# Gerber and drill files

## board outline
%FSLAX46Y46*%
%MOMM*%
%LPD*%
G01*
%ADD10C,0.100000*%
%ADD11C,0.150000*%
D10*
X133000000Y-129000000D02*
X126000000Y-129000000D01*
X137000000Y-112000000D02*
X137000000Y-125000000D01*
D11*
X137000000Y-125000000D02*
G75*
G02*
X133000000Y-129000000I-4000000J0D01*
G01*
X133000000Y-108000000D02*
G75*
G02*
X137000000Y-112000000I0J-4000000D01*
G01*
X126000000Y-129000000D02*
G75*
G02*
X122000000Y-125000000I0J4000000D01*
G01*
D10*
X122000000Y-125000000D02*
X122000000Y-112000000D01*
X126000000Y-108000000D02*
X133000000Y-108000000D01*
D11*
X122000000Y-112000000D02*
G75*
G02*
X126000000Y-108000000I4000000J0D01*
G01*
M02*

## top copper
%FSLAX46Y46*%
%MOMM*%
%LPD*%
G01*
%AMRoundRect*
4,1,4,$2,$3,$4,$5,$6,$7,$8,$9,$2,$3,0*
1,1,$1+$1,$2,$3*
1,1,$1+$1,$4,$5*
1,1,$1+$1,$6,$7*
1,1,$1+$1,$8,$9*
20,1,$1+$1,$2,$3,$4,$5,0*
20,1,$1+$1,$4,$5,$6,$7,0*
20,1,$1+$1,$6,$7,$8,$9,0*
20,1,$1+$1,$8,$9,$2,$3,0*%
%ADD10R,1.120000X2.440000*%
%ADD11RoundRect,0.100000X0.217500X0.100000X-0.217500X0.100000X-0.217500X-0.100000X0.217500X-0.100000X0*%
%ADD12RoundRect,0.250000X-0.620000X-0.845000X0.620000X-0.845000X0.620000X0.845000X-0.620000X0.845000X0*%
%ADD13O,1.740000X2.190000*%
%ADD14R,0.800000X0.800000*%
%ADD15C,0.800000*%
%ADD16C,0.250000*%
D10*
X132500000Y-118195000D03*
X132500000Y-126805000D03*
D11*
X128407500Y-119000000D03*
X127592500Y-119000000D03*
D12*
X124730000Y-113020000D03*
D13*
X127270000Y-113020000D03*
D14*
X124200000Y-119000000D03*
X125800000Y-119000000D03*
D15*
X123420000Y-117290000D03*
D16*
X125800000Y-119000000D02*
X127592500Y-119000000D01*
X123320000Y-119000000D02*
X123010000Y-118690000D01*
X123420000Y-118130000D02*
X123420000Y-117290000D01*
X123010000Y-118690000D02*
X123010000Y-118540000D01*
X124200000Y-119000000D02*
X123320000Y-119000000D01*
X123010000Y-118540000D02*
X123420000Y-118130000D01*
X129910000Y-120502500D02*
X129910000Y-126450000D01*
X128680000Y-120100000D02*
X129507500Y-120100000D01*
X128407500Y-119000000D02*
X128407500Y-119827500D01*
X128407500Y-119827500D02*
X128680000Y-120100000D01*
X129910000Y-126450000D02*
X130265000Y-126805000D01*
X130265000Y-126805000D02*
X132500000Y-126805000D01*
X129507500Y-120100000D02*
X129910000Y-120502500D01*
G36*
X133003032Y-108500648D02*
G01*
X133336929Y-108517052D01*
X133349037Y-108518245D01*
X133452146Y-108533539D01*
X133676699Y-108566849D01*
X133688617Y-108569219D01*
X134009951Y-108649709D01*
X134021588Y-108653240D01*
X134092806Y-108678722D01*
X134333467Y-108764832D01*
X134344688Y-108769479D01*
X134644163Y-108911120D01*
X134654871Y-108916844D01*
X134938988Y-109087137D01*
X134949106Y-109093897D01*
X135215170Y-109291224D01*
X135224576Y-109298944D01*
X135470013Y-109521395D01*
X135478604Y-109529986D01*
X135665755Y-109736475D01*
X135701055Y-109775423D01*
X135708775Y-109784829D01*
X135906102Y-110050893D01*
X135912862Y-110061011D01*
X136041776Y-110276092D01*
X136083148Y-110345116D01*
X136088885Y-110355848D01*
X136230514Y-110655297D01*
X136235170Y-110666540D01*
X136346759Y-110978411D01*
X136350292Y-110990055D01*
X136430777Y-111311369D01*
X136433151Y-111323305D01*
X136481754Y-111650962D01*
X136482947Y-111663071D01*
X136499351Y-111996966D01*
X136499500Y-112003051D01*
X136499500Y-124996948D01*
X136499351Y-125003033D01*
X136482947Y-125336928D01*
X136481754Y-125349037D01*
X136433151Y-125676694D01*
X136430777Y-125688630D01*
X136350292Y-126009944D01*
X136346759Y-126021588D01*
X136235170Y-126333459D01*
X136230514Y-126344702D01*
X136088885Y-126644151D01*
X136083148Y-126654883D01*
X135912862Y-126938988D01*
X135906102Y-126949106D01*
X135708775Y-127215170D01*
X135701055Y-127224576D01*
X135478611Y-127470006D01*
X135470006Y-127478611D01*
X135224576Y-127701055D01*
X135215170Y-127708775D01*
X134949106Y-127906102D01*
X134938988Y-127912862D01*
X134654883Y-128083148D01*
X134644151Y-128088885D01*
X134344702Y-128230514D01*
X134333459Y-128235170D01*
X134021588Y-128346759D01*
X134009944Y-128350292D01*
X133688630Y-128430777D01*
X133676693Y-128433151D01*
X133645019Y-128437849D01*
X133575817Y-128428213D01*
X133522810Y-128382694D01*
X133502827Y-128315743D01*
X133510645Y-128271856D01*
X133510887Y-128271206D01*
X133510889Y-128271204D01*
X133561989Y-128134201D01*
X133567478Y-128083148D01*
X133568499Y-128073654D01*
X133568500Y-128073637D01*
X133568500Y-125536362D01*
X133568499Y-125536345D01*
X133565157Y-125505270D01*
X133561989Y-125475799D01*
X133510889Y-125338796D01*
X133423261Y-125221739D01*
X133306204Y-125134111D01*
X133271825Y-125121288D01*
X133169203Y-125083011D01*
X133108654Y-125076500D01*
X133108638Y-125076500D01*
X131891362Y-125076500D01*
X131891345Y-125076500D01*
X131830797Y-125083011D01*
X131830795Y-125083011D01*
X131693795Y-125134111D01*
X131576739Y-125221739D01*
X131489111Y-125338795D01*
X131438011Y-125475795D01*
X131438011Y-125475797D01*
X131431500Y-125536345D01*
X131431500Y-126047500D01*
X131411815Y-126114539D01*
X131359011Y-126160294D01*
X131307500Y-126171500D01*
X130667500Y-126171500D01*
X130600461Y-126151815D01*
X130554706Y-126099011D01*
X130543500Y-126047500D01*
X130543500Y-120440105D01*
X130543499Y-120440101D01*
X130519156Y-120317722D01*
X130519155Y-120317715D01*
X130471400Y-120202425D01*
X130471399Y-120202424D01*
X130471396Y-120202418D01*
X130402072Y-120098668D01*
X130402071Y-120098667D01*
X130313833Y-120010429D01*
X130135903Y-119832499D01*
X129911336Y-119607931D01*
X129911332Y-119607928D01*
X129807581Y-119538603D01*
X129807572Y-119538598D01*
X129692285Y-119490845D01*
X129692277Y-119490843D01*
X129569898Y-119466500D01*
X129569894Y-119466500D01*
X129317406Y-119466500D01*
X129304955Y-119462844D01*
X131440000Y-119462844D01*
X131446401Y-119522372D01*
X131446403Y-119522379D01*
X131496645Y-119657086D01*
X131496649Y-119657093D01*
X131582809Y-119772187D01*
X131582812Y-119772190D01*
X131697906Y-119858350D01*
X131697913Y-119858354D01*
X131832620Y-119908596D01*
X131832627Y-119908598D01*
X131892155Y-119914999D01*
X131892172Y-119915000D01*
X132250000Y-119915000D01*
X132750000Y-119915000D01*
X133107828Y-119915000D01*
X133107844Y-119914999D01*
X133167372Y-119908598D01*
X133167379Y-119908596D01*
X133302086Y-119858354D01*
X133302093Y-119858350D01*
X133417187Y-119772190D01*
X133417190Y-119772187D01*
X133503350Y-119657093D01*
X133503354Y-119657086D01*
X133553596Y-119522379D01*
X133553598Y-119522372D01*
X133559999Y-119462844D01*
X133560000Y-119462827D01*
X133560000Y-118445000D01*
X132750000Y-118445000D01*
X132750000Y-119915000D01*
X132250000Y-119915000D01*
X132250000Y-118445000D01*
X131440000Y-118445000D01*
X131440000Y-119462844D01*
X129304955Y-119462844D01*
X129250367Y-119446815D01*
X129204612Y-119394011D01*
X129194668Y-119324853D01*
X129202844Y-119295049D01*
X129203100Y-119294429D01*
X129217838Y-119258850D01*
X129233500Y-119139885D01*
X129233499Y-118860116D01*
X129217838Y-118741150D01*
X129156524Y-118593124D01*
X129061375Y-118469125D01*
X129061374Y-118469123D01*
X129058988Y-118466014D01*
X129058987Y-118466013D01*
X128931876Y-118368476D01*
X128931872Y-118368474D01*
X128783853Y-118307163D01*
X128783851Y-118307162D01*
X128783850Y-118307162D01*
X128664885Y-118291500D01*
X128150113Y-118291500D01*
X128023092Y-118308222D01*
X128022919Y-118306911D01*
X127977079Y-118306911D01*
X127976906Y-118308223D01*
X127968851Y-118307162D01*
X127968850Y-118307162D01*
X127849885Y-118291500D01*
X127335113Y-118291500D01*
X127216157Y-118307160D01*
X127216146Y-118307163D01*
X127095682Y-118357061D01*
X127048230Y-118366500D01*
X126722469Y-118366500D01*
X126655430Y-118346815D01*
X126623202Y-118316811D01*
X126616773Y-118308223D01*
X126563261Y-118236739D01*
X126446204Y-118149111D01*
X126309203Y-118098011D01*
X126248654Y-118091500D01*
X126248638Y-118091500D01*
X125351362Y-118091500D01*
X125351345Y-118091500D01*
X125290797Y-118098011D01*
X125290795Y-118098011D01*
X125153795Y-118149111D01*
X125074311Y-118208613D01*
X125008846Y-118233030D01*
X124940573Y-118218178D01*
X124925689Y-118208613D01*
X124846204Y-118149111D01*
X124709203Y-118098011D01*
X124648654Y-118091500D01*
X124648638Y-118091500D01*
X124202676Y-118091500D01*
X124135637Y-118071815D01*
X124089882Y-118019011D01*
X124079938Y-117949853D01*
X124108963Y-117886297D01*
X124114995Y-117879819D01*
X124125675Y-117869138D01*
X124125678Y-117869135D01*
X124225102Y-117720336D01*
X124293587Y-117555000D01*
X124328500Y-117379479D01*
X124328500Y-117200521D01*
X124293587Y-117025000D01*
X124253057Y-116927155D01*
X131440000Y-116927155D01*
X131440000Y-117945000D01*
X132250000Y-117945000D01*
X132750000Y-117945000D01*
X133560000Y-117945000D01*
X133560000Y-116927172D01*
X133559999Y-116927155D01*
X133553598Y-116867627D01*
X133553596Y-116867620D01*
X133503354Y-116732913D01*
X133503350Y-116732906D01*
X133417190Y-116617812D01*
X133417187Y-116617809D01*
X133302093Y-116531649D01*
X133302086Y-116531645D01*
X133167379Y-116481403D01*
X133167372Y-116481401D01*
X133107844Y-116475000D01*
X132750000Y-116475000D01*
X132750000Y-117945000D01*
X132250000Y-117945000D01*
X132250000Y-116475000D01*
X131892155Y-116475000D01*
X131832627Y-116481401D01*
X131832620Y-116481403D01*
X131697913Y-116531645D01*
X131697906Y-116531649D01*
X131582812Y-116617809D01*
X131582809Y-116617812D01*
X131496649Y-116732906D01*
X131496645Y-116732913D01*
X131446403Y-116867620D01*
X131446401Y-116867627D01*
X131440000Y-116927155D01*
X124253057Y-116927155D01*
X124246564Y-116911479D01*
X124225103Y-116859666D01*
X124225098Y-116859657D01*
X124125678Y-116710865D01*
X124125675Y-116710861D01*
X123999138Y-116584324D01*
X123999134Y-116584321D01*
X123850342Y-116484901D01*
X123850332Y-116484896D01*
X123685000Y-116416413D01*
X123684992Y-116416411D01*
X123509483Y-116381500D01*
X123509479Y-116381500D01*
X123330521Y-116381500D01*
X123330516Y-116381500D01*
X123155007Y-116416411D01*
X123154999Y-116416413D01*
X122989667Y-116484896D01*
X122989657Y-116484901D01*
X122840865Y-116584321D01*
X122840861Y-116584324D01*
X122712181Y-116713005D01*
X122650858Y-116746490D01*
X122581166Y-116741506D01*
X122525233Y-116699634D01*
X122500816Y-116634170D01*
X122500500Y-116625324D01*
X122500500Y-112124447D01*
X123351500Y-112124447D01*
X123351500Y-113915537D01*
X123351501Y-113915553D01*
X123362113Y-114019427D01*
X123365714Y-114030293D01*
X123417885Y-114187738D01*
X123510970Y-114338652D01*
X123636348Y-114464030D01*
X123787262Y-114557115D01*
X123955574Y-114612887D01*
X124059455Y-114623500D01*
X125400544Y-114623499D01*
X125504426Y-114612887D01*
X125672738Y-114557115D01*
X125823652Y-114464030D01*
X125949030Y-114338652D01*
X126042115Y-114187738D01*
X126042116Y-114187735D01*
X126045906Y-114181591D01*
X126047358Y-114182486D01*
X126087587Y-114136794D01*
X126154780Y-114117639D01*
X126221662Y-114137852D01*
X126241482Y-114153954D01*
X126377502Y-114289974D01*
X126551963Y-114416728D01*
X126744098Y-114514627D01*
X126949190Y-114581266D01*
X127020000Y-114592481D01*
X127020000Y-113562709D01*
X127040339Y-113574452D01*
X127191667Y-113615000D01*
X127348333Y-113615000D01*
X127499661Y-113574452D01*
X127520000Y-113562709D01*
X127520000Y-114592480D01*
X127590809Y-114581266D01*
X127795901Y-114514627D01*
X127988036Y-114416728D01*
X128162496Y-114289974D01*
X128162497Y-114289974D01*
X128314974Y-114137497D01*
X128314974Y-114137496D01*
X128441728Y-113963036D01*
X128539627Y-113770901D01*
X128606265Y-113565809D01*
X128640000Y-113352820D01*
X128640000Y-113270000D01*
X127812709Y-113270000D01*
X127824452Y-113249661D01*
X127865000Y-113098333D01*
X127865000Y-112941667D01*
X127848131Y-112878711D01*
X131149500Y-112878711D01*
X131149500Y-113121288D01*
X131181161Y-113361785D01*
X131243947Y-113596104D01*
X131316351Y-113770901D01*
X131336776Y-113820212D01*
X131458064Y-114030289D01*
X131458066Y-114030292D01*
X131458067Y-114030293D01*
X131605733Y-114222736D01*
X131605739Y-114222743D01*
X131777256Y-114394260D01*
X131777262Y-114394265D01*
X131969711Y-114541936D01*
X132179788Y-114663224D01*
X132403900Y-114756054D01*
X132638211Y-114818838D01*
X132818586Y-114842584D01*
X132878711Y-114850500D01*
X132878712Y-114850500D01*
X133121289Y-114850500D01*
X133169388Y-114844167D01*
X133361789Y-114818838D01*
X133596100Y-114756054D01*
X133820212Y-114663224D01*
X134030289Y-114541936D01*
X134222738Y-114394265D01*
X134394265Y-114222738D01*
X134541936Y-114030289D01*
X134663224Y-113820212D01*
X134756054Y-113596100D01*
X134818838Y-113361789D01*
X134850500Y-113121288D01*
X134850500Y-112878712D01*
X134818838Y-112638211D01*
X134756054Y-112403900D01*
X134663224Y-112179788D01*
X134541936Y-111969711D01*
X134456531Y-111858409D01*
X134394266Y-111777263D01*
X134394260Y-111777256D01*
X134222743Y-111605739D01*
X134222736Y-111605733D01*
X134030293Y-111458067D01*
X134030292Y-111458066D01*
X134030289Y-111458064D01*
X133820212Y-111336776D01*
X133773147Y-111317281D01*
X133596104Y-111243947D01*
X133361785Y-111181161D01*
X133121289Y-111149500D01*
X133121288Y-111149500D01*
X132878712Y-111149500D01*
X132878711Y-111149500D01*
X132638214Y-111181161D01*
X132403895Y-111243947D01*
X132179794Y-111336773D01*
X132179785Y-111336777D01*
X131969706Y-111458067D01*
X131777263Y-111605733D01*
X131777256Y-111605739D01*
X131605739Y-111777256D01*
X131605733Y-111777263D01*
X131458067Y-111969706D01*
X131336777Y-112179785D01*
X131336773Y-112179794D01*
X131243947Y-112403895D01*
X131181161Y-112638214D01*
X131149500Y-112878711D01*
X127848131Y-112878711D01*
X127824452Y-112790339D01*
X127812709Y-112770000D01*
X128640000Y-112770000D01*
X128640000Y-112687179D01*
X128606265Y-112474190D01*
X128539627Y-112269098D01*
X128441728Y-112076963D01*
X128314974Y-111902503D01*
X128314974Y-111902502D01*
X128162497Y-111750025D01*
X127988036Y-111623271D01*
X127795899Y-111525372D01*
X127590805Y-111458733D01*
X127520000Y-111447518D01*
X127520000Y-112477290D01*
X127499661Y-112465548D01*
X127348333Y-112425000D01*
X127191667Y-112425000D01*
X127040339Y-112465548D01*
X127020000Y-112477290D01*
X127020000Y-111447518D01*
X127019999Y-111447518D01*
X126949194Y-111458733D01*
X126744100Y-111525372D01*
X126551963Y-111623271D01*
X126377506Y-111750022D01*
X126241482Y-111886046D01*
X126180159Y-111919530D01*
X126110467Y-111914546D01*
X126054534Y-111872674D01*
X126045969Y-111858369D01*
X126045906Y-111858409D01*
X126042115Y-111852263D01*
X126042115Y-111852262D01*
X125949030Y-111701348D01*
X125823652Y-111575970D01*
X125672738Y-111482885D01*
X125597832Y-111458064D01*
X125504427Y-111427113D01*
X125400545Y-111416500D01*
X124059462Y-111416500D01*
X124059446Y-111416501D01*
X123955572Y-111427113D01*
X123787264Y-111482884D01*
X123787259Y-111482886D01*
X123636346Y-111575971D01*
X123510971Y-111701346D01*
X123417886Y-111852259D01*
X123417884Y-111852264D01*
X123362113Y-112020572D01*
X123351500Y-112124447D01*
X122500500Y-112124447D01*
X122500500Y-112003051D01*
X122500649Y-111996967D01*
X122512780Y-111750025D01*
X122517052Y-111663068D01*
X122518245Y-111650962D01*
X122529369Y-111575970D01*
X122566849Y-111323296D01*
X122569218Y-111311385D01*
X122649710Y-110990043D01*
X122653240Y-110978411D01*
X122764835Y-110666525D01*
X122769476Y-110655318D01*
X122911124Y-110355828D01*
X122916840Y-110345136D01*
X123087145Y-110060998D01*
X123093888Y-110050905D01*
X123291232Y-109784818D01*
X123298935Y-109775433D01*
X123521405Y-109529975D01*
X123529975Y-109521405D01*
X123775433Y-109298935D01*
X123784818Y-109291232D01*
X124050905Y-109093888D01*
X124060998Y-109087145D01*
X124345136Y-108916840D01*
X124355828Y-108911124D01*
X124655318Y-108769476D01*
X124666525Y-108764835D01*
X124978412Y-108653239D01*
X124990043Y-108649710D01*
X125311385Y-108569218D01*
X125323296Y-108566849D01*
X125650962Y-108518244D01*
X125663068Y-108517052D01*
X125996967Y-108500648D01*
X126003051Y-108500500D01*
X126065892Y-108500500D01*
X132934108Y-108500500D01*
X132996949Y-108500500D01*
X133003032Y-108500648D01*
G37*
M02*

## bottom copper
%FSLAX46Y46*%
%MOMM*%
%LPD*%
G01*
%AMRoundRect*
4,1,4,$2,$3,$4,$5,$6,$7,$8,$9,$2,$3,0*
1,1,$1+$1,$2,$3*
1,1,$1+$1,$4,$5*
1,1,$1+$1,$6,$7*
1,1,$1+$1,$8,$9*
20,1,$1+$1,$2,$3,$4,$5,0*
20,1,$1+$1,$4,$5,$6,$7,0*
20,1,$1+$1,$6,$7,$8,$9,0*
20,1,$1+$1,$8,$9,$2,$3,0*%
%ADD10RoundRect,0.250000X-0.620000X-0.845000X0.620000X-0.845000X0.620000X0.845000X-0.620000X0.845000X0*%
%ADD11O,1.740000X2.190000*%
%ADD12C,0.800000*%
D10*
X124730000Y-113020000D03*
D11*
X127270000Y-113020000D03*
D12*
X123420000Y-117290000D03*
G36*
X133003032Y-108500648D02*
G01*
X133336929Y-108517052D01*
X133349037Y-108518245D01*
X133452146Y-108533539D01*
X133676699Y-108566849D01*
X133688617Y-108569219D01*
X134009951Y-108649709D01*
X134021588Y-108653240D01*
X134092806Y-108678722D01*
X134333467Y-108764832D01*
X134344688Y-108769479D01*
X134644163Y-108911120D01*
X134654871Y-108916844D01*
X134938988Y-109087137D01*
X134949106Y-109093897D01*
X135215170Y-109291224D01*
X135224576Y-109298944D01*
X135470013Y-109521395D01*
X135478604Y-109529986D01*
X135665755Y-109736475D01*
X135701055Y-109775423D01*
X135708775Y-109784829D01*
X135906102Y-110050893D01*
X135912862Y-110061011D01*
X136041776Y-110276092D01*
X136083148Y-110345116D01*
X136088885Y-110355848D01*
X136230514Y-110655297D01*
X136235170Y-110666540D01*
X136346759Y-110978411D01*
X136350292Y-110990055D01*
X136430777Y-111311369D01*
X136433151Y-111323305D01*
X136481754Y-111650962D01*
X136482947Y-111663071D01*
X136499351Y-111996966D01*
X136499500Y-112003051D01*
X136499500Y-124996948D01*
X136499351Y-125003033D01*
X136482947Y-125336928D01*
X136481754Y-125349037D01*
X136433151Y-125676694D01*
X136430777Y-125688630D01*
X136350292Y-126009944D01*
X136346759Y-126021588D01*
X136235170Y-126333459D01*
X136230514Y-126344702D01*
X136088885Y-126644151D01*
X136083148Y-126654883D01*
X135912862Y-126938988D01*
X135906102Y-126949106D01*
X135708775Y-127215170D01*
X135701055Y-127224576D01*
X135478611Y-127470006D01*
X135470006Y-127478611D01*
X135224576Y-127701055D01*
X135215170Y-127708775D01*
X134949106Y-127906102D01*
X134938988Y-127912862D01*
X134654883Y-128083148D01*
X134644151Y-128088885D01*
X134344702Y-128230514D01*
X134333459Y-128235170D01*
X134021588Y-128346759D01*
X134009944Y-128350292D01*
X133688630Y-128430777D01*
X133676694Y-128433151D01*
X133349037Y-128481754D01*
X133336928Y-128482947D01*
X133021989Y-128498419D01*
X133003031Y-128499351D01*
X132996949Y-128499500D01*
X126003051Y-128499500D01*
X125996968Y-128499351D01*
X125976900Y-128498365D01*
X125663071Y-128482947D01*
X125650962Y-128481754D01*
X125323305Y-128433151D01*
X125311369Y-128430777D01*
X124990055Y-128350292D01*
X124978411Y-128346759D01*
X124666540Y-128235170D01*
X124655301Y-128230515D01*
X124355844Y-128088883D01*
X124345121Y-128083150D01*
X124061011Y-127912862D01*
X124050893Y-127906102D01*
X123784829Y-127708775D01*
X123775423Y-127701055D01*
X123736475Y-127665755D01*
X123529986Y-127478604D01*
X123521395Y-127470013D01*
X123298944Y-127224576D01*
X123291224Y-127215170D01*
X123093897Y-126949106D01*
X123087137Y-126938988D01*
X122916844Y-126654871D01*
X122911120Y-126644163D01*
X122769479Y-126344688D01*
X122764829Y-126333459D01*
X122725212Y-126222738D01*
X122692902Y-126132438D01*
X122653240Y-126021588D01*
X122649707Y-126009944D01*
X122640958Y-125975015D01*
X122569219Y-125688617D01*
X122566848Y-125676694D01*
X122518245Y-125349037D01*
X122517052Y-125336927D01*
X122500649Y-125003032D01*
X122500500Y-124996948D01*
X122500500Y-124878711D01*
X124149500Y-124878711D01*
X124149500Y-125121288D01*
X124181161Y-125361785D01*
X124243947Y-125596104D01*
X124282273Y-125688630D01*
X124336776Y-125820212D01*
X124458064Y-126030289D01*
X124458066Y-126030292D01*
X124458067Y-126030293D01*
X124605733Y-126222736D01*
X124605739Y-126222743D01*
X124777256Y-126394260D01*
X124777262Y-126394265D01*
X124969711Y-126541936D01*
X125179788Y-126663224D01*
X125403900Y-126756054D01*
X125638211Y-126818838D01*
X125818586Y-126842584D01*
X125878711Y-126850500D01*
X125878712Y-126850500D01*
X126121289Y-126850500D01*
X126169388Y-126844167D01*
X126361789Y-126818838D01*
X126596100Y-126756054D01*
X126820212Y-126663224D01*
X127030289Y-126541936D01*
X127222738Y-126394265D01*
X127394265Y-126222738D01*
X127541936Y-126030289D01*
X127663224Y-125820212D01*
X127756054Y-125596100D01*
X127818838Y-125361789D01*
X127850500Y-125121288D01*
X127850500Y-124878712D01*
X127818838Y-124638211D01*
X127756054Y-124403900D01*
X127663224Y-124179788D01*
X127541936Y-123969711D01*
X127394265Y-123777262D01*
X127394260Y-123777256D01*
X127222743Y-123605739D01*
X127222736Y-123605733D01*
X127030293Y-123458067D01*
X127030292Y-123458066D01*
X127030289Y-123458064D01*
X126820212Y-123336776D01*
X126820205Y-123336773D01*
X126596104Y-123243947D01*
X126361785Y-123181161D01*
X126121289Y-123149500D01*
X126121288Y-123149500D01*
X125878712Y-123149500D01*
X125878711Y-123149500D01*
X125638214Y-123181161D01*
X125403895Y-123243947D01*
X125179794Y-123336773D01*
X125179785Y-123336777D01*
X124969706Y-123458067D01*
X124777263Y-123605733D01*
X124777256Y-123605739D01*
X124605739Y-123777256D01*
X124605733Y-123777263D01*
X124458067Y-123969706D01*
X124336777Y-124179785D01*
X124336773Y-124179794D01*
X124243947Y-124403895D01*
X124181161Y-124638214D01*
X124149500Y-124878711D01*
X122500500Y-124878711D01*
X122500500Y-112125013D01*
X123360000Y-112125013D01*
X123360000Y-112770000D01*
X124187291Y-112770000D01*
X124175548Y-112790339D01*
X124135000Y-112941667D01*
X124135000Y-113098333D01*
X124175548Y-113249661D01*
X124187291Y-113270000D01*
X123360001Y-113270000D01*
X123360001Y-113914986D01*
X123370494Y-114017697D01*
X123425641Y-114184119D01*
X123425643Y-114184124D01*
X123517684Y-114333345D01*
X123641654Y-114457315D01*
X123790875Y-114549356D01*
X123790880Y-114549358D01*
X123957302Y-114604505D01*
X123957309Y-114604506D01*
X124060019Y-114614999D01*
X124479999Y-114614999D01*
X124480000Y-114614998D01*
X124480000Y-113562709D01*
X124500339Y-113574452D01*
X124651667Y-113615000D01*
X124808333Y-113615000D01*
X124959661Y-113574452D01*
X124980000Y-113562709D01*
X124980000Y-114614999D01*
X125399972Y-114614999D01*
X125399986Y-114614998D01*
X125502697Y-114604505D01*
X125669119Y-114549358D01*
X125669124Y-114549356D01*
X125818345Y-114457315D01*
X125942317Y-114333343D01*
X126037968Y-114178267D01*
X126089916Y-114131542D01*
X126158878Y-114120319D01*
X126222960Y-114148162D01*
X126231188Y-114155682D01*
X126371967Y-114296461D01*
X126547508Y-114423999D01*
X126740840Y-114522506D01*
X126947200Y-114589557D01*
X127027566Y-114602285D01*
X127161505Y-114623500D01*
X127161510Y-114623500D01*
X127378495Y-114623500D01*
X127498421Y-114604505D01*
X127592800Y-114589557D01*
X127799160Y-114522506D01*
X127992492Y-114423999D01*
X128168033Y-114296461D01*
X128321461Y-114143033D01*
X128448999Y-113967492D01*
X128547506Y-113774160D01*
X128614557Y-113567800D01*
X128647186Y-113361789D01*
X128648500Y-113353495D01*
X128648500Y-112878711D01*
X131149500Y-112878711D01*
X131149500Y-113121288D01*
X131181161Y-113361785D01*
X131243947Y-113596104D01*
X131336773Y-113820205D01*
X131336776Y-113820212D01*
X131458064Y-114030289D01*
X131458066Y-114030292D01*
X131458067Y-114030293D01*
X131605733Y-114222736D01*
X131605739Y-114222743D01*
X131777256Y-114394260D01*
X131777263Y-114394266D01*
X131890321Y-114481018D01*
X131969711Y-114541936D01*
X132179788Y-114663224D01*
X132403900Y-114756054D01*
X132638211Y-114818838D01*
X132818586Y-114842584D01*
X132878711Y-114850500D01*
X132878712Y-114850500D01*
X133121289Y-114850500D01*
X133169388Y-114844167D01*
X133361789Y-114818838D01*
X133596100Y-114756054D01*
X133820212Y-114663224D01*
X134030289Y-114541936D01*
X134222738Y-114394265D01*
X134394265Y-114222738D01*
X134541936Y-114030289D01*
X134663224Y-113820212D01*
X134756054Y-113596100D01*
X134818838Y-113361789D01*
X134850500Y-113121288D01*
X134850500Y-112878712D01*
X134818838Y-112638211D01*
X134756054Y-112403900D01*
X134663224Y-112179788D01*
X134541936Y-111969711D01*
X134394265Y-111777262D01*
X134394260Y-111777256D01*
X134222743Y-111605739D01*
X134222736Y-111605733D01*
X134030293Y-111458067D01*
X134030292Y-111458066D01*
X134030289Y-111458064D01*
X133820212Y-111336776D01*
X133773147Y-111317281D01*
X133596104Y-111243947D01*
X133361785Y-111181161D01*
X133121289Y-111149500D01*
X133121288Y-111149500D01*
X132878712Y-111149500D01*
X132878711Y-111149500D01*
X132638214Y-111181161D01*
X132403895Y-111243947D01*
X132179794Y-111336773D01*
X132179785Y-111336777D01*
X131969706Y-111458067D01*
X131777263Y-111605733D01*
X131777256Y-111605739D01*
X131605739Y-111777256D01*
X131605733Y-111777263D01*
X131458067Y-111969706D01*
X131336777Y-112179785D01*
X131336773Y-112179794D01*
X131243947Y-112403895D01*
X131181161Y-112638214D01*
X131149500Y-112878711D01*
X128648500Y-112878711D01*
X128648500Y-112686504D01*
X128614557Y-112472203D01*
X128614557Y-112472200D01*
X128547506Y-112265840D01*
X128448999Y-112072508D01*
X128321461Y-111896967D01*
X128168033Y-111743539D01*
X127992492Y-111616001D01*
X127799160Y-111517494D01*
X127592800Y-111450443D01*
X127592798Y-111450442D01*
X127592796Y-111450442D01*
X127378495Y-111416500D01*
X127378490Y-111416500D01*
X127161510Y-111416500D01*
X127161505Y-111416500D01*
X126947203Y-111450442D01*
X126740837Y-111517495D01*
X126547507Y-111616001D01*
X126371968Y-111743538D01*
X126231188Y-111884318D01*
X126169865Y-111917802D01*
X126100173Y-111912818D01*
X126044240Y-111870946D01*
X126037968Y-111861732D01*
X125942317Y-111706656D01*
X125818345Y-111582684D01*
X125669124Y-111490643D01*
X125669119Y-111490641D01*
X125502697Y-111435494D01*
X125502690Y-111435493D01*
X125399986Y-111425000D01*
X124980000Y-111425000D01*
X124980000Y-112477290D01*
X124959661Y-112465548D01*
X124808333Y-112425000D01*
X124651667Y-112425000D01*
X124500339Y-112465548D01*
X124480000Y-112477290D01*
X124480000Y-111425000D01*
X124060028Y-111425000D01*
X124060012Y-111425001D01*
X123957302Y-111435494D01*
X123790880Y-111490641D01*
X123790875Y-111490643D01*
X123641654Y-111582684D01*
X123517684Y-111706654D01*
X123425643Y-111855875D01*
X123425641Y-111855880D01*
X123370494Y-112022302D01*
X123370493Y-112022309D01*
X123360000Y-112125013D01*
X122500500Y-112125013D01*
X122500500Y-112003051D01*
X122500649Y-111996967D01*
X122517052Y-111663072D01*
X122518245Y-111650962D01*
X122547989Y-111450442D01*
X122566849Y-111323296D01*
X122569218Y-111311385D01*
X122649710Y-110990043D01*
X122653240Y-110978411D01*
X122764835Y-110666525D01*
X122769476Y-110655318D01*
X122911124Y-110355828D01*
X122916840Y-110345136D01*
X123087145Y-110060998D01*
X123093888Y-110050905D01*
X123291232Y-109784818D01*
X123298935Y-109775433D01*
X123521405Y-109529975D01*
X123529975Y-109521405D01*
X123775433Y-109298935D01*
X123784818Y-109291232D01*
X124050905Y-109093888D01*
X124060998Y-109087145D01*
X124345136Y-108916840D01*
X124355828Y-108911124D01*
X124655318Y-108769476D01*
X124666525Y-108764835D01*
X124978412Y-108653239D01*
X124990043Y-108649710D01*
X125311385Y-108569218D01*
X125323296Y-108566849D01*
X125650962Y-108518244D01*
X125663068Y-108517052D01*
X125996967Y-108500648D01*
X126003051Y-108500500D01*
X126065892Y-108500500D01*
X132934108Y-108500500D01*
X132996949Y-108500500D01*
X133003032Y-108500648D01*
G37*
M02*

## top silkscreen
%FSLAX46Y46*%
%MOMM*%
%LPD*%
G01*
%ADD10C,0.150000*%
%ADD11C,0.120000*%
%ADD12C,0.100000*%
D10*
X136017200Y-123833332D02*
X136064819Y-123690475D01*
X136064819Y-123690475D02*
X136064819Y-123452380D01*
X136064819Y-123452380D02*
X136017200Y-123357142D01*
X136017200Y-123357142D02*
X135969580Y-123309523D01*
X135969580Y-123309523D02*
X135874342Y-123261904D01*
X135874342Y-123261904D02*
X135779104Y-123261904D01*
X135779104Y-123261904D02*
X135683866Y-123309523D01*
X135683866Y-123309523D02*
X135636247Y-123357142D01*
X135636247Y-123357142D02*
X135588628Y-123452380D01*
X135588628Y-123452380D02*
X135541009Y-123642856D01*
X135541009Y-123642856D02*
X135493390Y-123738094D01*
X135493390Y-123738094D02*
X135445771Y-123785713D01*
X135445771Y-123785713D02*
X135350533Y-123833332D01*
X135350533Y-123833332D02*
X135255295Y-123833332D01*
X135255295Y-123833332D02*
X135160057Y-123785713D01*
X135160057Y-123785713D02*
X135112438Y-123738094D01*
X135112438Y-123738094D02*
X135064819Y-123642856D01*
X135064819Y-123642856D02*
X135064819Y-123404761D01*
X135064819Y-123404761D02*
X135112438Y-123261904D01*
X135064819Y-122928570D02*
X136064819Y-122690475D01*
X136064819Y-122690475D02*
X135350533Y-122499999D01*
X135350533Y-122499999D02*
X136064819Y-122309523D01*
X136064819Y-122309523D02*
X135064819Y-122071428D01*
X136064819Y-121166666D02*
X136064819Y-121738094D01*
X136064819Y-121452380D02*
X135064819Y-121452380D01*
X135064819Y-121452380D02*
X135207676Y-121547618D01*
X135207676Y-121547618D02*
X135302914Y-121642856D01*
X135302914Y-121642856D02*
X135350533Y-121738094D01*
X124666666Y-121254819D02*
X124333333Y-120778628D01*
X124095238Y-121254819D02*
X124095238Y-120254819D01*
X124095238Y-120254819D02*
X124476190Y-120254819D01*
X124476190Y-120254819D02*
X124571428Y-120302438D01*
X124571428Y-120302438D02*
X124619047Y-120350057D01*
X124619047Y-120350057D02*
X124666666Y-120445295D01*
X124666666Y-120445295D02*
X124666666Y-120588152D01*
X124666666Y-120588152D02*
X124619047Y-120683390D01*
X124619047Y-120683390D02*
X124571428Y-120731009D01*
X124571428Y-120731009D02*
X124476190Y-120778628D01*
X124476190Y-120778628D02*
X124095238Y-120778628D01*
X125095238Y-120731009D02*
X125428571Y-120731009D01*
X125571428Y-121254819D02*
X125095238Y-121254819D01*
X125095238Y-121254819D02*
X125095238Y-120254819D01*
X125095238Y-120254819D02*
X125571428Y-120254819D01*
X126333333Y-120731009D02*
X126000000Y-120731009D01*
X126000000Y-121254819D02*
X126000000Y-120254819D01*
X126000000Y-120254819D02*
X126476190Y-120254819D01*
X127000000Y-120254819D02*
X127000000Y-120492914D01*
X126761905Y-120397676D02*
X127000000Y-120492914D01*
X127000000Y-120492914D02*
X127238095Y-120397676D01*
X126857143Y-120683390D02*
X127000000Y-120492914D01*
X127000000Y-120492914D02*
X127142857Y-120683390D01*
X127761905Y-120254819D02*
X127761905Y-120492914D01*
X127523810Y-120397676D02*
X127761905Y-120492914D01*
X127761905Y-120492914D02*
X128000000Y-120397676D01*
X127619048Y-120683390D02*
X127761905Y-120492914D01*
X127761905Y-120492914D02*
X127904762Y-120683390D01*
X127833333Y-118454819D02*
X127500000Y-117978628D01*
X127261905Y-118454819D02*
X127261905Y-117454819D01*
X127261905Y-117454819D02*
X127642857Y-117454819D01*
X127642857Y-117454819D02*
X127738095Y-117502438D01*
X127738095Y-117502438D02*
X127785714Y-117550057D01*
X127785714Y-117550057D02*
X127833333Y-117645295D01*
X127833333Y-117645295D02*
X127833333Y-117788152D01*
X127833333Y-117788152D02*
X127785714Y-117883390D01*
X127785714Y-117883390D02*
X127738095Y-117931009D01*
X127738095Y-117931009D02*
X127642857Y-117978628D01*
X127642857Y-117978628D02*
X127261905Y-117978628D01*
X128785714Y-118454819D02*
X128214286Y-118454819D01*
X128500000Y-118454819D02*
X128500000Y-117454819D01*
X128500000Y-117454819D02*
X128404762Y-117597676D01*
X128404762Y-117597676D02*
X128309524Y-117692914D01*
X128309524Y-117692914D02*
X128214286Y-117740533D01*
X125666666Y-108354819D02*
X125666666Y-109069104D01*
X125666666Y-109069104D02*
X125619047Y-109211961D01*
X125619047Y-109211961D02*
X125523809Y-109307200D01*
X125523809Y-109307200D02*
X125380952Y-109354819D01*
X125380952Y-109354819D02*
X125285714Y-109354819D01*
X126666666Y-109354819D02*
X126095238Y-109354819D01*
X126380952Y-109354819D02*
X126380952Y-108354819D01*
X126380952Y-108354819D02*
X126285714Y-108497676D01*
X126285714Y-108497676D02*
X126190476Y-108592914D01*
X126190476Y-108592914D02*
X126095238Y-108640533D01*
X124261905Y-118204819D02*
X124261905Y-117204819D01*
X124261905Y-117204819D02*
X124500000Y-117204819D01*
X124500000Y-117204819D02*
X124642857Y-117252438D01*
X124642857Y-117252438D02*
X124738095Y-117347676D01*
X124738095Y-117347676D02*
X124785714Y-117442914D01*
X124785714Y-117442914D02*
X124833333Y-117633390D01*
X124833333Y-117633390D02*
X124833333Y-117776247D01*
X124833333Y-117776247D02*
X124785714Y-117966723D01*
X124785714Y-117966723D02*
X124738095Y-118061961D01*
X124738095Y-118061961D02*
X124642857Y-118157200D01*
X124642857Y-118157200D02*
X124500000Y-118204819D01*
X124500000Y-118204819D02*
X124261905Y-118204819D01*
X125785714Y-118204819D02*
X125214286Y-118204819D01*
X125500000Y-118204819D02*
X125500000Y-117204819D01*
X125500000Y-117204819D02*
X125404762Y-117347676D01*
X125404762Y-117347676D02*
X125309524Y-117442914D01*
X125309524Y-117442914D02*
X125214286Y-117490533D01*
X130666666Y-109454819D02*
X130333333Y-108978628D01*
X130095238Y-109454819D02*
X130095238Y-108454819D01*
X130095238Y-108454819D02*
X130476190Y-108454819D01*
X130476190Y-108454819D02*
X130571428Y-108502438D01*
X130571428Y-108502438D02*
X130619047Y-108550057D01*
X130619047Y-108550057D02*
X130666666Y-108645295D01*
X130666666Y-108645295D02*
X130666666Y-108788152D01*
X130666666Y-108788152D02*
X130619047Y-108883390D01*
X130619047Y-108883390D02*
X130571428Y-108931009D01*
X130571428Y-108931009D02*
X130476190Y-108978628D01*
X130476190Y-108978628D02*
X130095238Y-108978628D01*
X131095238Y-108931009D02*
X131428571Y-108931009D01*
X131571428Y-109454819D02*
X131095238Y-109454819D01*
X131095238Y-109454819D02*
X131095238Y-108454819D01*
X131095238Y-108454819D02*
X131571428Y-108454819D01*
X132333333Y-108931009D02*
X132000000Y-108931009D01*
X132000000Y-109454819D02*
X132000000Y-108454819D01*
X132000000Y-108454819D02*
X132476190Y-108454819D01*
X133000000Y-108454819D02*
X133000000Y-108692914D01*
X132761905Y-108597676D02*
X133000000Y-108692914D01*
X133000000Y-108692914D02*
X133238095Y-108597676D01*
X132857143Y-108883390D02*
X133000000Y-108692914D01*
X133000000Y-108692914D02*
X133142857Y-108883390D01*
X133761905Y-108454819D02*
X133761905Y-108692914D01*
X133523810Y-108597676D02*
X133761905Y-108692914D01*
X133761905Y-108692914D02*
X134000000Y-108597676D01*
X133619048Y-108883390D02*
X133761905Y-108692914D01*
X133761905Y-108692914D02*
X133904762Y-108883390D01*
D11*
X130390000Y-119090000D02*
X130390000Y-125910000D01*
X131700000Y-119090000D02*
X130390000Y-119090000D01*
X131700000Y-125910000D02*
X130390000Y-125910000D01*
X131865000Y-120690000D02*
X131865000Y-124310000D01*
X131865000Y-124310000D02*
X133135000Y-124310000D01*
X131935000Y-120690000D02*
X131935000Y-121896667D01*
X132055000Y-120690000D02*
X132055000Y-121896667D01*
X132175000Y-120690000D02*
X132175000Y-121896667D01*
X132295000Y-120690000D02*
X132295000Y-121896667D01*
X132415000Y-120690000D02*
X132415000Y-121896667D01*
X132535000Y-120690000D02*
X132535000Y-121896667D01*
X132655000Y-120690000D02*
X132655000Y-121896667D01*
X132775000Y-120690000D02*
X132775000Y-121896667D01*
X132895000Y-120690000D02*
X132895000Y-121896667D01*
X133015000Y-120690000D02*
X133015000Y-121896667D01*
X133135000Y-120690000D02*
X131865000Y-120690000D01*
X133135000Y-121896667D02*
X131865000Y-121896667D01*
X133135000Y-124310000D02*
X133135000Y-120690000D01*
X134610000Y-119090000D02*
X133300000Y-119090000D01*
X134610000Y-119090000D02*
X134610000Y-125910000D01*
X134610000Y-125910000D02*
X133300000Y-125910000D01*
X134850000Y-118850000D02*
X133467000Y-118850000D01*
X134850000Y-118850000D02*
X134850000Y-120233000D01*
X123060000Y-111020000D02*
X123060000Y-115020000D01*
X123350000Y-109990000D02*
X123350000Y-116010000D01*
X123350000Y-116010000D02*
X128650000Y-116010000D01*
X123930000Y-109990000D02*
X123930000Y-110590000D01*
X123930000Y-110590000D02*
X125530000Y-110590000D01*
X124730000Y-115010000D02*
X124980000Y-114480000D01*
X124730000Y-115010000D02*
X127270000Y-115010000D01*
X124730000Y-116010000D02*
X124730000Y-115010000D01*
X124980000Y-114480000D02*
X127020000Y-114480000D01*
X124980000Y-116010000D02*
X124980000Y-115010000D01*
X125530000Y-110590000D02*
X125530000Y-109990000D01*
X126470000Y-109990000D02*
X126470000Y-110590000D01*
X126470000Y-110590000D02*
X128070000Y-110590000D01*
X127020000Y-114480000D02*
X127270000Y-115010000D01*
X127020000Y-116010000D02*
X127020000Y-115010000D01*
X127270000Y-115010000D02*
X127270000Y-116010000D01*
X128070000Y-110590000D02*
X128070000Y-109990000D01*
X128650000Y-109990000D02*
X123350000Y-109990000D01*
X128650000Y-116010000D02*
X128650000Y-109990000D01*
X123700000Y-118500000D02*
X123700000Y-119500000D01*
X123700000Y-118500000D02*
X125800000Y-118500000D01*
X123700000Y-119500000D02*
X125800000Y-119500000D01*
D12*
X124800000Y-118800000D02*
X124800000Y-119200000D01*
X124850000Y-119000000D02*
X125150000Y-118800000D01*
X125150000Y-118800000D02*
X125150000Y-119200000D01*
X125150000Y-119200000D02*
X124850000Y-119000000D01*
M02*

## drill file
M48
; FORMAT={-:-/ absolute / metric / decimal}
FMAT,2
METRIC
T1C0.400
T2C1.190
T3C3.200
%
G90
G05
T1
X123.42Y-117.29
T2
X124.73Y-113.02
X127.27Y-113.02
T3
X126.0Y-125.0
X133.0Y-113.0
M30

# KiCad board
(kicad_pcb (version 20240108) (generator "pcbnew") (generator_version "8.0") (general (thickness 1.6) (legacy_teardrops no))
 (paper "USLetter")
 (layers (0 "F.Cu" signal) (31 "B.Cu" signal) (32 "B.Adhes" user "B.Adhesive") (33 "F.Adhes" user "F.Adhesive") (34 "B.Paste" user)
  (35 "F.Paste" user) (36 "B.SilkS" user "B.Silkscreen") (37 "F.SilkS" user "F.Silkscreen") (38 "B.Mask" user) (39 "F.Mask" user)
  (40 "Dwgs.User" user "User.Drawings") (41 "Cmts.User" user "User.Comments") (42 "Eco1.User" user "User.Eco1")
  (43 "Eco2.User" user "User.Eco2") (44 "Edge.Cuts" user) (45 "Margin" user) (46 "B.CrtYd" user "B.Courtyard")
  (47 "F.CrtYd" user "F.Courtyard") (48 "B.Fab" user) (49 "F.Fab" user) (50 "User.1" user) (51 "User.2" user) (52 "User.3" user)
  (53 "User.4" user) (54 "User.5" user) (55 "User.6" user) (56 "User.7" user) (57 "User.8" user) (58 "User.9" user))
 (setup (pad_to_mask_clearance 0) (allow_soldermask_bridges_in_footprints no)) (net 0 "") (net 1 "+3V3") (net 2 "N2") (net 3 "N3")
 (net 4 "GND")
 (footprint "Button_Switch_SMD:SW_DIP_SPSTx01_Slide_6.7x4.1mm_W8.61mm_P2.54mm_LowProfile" (layer "F.Cu") (at 132.5 122.5 -90)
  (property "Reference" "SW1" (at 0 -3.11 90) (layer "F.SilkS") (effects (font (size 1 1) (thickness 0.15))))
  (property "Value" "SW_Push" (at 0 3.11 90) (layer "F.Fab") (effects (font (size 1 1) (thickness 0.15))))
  (fp_line (start -3.41 2.11) (end 3.41 2.11) (stroke (width 0.12) (type solid)) (layer "F.SilkS"))
  (fp_line (start -3.41 0.8) (end -3.41 2.11) (stroke (width 0.12) (type solid)) (layer "F.SilkS"))
  (fp_line (start 3.41 0.8) (end 3.41 2.11) (stroke (width 0.12) (type solid)) (layer "F.SilkS"))
  (fp_line (start -1.81 0.635) (end 1.81 0.635) (stroke (width 0.12) (type solid)) (layer "F.SilkS"))
  (fp_line (start 1.81 0.635) (end 1.81 -0.635) (stroke (width 0.12) (type solid)) (layer "F.SilkS"))
  (fp_line (start -1.81 0.565) (end -0.603333 0.565) (stroke (width 0.12) (type solid)) (layer "F.SilkS"))
  (fp_line (start -1.81 0.445) (end -0.603333 0.445) (stroke (width 0.12) (type solid)) (layer "F.SilkS"))
  (fp_line (start -1.81 0.325) (end -0.603333 0.325) (stroke (width 0.12) (type solid)) (layer "F.SilkS"))
  (fp_line (start -1.81 0.205) (end -0.603333 0.205) (stroke (width 0.12) (type solid)) (layer "F.SilkS"))
  (fp_line (start -1.81 0.085) (end -0.603333 0.085) (stroke (width 0.12) (type solid)) (layer "F.SilkS"))
  (fp_line (start -1.81 -0.035) (end -0.603333 -0.035) (stroke (width 0.12) (type solid)) (layer "F.SilkS"))
  (fp_line (start -1.81 -0.155) (end -0.603333 -0.155) (stroke (width 0.12) (type solid)) (layer "F.SilkS"))
  (fp_line (start -1.81 -0.275) (end -0.603333 -0.275) (stroke (width 0.12) (type solid)) (layer "F.SilkS"))
  (fp_line (start -1.81 -0.395) (end -0.603333 -0.395) (stroke (width 0.12) (type solid)) (layer "F.SilkS"))
  (fp_line (start -1.81 -0.515) (end -0.603333 -0.515) (stroke (width 0.12) (type solid)) (layer "F.SilkS"))
  (fp_line (start -1.81 -0.635) (end -1.81 0.635) (stroke (width 0.12) (type solid)) (layer "F.SilkS"))
  (fp_line (start -0.603333 -0.635) (end -0.603333 0.635) (stroke (width 0.12) (type solid)) (layer "F.SilkS"))
  (fp_line (start 1.81 -0.635) (end -1.81 -0.635) (stroke (width 0.12) (type solid)) (layer "F.SilkS"))
  (fp_line (start -3.41 -2.11) (end -3.41 -0.8) (stroke (width 0.12) (type solid)) (layer "F.SilkS"))
  (fp_line (start -3.41 -2.11) (end 3.41 -2.11) (stroke (width 0.12) (type solid)) (layer "F.SilkS"))
  (fp_line (start 3.41 -2.11) (end 3.41 -0.8) (stroke (width 0.12) (type solid)) (layer "F.SilkS"))
  (fp_line (start -3.65 -2.35) (end -3.65 -0.967) (stroke (width 0.12) (type solid)) (layer "F.SilkS"))
  (fp_line (start -3.65 -2.35) (end -2.267 -2.35) (stroke (width 0.12) (type solid)) (layer "F.SilkS"))
  (pad "1" smd rect (at -4.305 0 270) (size 2.44 1.12) (layers "F.Cu" "F.Paste" "F.Mask") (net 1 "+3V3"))
  (pad "2" smd rect (at 4.305 0 270) (size 2.44 1.12) (layers "F.Cu" "F.Paste" "F.Mask") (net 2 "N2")))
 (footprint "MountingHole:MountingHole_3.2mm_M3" (layer "F.Cu") (at 126 125)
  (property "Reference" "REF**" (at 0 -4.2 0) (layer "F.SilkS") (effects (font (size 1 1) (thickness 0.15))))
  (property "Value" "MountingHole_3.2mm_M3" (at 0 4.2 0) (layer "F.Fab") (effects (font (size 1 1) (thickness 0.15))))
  (pad "" np_thru_hole circle (at 0 0) (size 3.2 3.2) (drill 3.2) (layers "*.Cu" "*.Mask")))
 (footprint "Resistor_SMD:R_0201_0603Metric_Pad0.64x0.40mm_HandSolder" (layer "F.Cu") (at 128 119 180)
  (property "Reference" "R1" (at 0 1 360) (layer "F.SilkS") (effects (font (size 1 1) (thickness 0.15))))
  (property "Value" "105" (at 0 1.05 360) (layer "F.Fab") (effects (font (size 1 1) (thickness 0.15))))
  (pad "" smd roundrect (at -0.4325 0 180) (size 0.458 0.36) (layers "F.Paste") (roundrect_rratio 0.25))
  (pad "" smd roundrect (at 0.4325 0 180) (size 0.458 0.36) (layers "F.Paste") (roundrect_rratio 0.25))
  (pad "1" smd roundrect (at -0.4075 0 180) (size 0.635 0.4) (layers "F.Cu" "F.Mask") (roundrect_rratio 0.25) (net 2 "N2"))
  (pad "2" smd roundrect (at 0.4075 0 180) (size 0.635 0.4) (layers "F.Cu" "F.Mask") (roundrect_rratio 0.25) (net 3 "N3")))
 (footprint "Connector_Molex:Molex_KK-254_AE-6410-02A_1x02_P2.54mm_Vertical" (layer "F.Cu") (at 124.73 113.02)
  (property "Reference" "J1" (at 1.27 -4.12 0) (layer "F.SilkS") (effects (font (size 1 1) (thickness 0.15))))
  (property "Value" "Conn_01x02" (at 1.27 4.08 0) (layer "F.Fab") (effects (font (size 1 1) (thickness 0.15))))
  (fp_line (start -1.67 -2) (end -1.67 2) (stroke (width 0.12) (type solid)) (layer "F.SilkS"))
  (fp_line (start -1.38 -3.03) (end -1.38 2.99) (stroke (width 0.12) (type solid)) (layer "F.SilkS"))
  (fp_line (start -1.38 2.99) (end 3.92 2.99) (stroke (width 0.12) (type solid)) (layer "F.SilkS"))
  (fp_line (start -0.8 -3.03) (end -0.8 -2.43) (stroke (width 0.12) (type solid)) (layer "F.SilkS"))
  (fp_line (start -0.8 -2.43) (end 0.8 -2.43) (stroke (width 0.12) (type solid)) (layer "F.SilkS"))
  (fp_line (start 0 1.99) (end 0.25 1.46) (stroke (width 0.12) (type solid)) (layer "F.SilkS"))
  (fp_line (start 0 1.99) (end 2.54 1.99) (stroke (width 0.12) (type solid)) (layer "F.SilkS"))
  (fp_line (start 0 2.99) (end 0 1.99) (stroke (width 0.12) (type solid)) (layer "F.SilkS"))
  (fp_line (start 0.25 1.46) (end 2.29 1.46) (stroke (width 0.12) (type solid)) (layer "F.SilkS"))
  (fp_line (start 0.25 2.99) (end 0.25 1.99) (stroke (width 0.12) (type solid)) (layer "F.SilkS"))
  (fp_line (start 0.8 -2.43) (end 0.8 -3.03) (stroke (width 0.12) (type solid)) (layer "F.SilkS"))
  (fp_line (start 1.74 -3.03) (end 1.74 -2.43) (stroke (width 0.12) (type solid)) (layer "F.SilkS"))
  (fp_line (start 1.74 -2.43) (end 3.34 -2.43) (stroke (width 0.12) (type solid)) (layer "F.SilkS"))
  (fp_line (start 2.29 1.46) (end 2.54 1.99) (stroke (width 0.12) (type solid)) (layer "F.SilkS"))
  (fp_line (start 2.29 2.99) (end 2.29 1.99) (stroke (width 0.12) (type solid)) (layer "F.SilkS"))
  (fp_line (start 2.54 1.99) (end 2.54 2.99) (stroke (width 0.12) (type solid)) (layer "F.SilkS"))
  (fp_line (start 3.34 -2.43) (end 3.34 -3.03) (stroke (width 0.12) (type solid)) (layer "F.SilkS"))
  (fp_line (start 3.92 -3.03) (end -1.38 -3.03) (stroke (width 0.12) (type solid)) (layer "F.SilkS"))
  (fp_line (start 3.92 2.99) (end 3.92 -3.03) (stroke (width 0.12) (type solid)) (layer "F.SilkS"))
  (pad "1" thru_hole roundrect (at 0 0) (size 1.74 2.19) (drill 1.19) (layers "*.Cu" "*.Mask") (remove_unused_layers no)
   (roundrect_rratio 0.143678) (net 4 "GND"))
  (pad "2" thru_hole oval (at 2.54 0) (size 1.74 2.19) (drill 1.19) (layers "*.Cu" "*.Mask") (remove_unused_layers no) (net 1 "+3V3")))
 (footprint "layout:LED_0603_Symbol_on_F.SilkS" (layer "F.Cu") (at 125 119)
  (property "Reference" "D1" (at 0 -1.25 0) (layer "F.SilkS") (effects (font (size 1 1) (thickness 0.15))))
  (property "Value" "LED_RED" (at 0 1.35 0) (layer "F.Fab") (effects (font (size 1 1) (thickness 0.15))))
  (fp_line (start -1.3 -0.5) (end -1.3 0.5) (stroke (width 0.12) (type solid)) (layer "F.SilkS"))
  (fp_line (start -1.3 -0.5) (end 0.8 -0.5) (stroke (width 0.12) (type solid)) (layer "F.SilkS"))
  (fp_line (start -1.3 0.5) (end 0.8 0.5) (stroke (width 0.12) (type solid)) (layer "F.SilkS"))
  (fp_line (start -0.2 -0.2) (end -0.2 0.2) (stroke (width 0.1) (type solid)) (layer "F.SilkS"))
  (fp_line (start -0.15 0) (end 0.15 -0.2) (stroke (width 0.1) (type solid)) (layer "F.SilkS"))
  (fp_line (start 0.15 -0.2) (end 0.15 0.2) (stroke (width 0.1) (type solid)) (layer "F.SilkS"))
  (fp_line (start 0.15 0.2) (end -0.15 0) (stroke (width 0.1) (type solid)) (layer "F.SilkS"))
  (pad "1" smd rect (at -0.8 0 180) (size 0.8 0.8) (layers "F.Cu" "F.Paste" "F.Mask") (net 4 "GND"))
  (pad "2" smd rect (at 0.8 0 180) (size 0.8 0.8) (layers "F.Cu" "F.Paste" "F.Mask") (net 3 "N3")))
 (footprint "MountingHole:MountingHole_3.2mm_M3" (layer "F.Cu") (at 133 113)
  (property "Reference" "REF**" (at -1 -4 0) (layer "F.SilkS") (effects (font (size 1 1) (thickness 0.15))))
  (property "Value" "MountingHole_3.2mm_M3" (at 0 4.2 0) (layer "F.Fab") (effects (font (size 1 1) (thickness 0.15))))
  (pad "" np_thru_hole circle (at 0 0) (size 3.2 3.2) (drill 3.2) (layers "*.Cu" "*.Mask")))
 (gr_line (start 133 129) (end 126 129) (stroke (width 0.1) (type default)) (layer "Edge.Cuts"))
 (gr_line (start 137 112) (end 137 125) (stroke (width 0.1) (type default)) (layer "Edge.Cuts"))
 (gr_arc (start 137 125) (mid 135.828427 127.828427) (end 133 129) (stroke (width 0.15) (type default)) (layer "Edge.Cuts"))
 (gr_arc (start 133 108) (mid 135.828427 109.171573) (end 137 112) (stroke (width 0.15) (type default)) (layer "Edge.Cuts"))
 (gr_arc (start 126 129) (mid 123.171573 127.828427) (end 122 125) (stroke (width 0.15) (type default)) (layer "Edge.Cuts"))
 (gr_line (start 122 125) (end 122 112) (stroke (width 0.1) (type default)) (layer "Edge.Cuts"))
 (gr_line (start 126 108) (end 133 108) (stroke (width 0.1) (type default)) (layer "Edge.Cuts"))
 (gr_arc (start 122 112) (mid 123.171573 109.171573) (end 126 108) (stroke (width 0.15) (type default)) (layer "Edge.Cuts"))
 (segment (start 125.8 119) (end 127.5925 119) (width 0.25) (layer "F.Cu") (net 3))
 (segment (start 123.32 119) (end 123.01 118.69) (width 0.25) (layer "F.Cu") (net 4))
 (segment (start 123.42 118.13) (end 123.42 117.29) (width 0.25) (layer "F.Cu") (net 4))
 (segment (start 123.01 118.69) (end 123.01 118.54) (width 0.25) (layer "F.Cu") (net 4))
 (segment (start 124.2 119) (end 123.32 119) (width 0.25) (layer "F.Cu") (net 4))
 (segment (start 123.01 118.54) (end 123.42 118.13) (width 0.25) (layer "F.Cu") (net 4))
 (via (at 123.42 117.29) (size 0.8) (drill 0.4) (layers "F.Cu" "B.Cu") (free yes) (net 4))
 (segment (start 129.91 120.5025) (end 129.91 126.45) (width 0.25) (layer "F.Cu") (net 2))
 (segment (start 128.68 120.1) (end 129.5075 120.1) (width 0.25) (layer "F.Cu") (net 2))
 (segment (start 128.4075 119) (end 128.4075 119.8275) (width 0.25) (layer "F.Cu") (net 2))
 (segment (start 128.4075 119.8275) (end 128.68 120.1) (width 0.25) (layer "F.Cu") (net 2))
 (segment (start 129.91 126.45) (end 130.265 126.805) (width 0.25) (layer "F.Cu") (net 2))
 (segment (start 130.265 126.805) (end 132.5 126.805) (width 0.25) (layer "F.Cu") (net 2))
 (segment (start 129.5075 120.1) (end 129.91 120.5025) (width 0.25) (layer "F.Cu") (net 2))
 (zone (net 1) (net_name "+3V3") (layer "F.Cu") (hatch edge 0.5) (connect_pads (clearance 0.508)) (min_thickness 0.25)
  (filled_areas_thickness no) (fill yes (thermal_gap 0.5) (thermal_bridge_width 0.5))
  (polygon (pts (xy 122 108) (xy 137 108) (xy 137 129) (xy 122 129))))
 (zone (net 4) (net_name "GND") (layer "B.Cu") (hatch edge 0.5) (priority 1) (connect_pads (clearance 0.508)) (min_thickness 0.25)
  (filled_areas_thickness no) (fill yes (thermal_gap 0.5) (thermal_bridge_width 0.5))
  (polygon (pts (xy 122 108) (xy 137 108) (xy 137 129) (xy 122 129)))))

